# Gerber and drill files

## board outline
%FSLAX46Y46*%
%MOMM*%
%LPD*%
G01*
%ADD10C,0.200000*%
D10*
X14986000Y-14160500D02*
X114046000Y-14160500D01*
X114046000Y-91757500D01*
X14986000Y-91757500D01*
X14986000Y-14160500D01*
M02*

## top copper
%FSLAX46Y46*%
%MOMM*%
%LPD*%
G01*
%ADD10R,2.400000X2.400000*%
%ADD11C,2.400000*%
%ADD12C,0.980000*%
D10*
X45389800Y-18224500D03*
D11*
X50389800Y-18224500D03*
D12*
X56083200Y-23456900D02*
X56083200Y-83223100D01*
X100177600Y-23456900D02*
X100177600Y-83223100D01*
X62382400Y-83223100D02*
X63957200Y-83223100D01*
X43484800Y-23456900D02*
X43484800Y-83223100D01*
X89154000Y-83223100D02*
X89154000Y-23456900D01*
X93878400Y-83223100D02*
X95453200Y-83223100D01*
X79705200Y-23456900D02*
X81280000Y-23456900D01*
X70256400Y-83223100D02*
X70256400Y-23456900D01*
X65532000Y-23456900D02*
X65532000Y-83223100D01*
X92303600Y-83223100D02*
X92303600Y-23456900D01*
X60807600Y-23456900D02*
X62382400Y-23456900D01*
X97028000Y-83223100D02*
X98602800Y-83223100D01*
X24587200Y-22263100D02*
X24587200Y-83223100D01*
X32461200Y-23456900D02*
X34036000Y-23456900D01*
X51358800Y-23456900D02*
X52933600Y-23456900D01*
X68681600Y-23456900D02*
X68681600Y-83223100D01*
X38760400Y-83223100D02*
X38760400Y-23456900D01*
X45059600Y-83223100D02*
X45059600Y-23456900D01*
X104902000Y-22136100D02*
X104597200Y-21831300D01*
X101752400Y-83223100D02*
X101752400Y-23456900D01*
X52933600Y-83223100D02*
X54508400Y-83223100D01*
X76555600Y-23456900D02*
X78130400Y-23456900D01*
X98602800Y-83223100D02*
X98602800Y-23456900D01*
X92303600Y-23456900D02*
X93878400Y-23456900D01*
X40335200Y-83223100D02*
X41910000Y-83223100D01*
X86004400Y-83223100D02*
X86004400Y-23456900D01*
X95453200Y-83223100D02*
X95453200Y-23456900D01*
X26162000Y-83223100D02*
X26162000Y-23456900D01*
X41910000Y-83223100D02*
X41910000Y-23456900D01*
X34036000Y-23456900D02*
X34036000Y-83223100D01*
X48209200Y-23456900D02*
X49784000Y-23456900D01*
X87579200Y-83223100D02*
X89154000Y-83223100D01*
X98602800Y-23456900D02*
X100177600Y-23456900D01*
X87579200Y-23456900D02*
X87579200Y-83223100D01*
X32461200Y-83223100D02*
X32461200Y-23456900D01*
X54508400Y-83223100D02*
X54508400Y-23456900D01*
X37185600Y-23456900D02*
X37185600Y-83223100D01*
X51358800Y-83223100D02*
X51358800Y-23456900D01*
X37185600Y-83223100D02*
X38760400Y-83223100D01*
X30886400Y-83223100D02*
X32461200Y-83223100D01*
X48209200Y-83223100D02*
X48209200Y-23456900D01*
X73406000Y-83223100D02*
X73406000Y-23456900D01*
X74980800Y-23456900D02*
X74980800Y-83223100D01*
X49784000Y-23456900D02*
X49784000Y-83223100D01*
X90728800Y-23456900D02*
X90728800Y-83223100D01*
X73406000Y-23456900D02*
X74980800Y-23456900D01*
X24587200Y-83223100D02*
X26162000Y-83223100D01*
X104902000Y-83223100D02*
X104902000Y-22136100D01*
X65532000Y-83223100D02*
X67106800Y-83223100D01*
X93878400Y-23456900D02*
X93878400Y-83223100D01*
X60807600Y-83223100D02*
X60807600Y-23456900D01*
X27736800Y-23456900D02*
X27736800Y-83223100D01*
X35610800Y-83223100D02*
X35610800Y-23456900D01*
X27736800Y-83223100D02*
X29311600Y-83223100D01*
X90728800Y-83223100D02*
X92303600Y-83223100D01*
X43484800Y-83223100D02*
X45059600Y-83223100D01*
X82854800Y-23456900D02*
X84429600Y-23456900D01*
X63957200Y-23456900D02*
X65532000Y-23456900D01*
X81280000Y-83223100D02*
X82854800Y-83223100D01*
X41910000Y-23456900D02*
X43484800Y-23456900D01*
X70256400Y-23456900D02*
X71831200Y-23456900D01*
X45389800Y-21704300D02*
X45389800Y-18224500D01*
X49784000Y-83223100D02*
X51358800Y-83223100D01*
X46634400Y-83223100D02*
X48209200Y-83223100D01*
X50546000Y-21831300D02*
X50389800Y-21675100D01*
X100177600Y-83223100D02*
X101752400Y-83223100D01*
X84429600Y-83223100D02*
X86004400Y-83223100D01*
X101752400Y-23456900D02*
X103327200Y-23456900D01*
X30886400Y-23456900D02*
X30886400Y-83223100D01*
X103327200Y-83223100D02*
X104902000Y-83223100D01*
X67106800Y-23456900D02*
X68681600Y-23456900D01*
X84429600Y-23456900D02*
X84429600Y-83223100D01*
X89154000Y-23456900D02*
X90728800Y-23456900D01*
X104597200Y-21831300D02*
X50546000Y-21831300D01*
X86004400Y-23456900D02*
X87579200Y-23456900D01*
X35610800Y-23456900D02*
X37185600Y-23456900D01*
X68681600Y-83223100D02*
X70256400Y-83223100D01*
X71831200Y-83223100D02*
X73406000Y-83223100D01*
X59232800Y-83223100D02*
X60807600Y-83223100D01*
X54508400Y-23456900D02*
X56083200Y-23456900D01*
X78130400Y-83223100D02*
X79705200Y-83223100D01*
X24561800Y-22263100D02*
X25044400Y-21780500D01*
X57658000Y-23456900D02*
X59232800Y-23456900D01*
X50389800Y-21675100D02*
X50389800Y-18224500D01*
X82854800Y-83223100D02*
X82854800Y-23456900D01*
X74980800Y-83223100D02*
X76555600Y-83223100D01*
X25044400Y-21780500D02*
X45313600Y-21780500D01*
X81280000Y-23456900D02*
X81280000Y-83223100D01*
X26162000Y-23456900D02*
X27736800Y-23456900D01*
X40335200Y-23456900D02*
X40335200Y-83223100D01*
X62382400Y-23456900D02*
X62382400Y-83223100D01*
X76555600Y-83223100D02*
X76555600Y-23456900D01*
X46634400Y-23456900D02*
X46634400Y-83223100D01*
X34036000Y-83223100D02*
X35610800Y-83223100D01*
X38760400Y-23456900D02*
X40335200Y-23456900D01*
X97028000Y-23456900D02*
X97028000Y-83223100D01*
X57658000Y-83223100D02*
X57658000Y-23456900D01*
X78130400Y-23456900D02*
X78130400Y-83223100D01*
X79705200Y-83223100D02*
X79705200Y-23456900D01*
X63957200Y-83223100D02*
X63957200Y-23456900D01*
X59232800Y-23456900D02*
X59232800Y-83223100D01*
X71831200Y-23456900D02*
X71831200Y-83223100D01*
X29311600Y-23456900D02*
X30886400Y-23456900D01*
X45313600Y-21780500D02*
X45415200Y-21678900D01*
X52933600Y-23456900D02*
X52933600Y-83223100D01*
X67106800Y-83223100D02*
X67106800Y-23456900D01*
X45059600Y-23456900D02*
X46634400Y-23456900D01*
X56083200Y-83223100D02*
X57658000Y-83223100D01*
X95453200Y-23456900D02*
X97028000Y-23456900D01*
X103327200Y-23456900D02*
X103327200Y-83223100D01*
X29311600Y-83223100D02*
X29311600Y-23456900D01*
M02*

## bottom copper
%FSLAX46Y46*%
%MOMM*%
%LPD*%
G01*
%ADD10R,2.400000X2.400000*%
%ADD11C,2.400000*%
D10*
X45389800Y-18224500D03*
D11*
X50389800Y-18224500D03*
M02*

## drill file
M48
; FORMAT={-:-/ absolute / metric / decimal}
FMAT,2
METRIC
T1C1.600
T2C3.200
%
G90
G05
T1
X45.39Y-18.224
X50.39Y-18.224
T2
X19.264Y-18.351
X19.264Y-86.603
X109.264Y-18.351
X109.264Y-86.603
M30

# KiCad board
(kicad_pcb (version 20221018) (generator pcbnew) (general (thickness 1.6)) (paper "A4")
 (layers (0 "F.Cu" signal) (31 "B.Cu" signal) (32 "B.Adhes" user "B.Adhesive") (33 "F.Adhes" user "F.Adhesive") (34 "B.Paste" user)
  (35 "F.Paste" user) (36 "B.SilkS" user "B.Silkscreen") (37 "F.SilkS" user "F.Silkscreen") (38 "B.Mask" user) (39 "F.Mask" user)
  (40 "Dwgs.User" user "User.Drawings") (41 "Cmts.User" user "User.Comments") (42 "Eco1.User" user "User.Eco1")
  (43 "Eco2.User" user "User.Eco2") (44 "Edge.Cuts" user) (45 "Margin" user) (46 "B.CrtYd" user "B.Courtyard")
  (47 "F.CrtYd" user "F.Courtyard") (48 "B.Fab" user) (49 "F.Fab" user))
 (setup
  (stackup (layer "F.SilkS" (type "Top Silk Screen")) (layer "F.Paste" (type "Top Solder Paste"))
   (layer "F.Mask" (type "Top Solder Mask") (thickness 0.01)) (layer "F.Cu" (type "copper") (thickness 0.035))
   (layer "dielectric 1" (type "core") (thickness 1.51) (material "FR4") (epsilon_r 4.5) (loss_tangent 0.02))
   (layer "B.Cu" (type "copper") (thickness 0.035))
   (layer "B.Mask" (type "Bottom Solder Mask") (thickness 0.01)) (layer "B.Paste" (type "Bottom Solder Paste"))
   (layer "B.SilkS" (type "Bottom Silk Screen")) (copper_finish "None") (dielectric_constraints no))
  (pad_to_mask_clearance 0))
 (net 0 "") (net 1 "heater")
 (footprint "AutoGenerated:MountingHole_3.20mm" (layer "F.Cu") (at 99.264 70.6035)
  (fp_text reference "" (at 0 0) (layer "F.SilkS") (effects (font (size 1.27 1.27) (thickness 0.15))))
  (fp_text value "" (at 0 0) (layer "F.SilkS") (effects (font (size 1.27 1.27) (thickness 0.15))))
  (pad "" np_thru_hole circle (at 10 16) (size 3.2 3.2) (drill 3.2) (layers "F&B.Cu" "*.Mask")))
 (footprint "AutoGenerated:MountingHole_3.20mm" (layer "F.Cu") (at 19.264 18.3515)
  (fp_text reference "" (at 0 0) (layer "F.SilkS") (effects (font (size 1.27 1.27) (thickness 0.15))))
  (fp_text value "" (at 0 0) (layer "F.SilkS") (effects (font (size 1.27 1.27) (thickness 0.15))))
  (pad "" np_thru_hole circle (at 0 0) (size 3.2 3.2) (drill 3.2) (layers "*.Cu" "*.Mask")))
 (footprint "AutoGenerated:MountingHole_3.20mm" (layer "F.Cu") (at 99.264 18.3515)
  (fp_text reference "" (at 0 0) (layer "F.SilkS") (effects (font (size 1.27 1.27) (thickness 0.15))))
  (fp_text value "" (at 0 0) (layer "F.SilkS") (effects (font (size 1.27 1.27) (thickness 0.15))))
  (pad "" np_thru_hole circle (at 10 0) (size 3.2 3.2) (drill 3.2) (layers "F&B.Cu" "*.Mask")))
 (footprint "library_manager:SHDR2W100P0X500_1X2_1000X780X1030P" (layer "F.Cu") (at 45.3898 18.2245)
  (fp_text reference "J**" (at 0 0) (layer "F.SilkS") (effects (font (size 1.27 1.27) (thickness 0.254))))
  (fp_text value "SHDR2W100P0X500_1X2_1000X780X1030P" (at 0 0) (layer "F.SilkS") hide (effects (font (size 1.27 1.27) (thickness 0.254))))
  (pad "1" thru_hole rect (at 0 0) (size 2.4 2.4) (drill 1.6) (layers "*.Cu" "*.Mask") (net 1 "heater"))
  (pad "2" thru_hole circle (at 5 0) (size 2.4 2.4) (drill 1.6) (layers "*.Cu" "*.Mask") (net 1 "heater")))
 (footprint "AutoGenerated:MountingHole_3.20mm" (layer "F.Cu") (at 19.264 70.6035)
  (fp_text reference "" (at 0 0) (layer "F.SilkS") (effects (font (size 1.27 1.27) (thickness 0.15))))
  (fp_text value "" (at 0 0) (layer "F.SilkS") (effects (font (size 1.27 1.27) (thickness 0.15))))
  (pad "" np_thru_hole circle (at 0 16) (size 3.2 3.2) (drill 3.2) (layers "F&B.Cu" "*.Mask")))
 (gr_rect (start 14.986 14.1605) (end 114.046 91.7575) (stroke (width 0.2) (type solid)) (fill none) (layer "Edge.Cuts"))
 (segment (start 56.0832 23.4569) (end 56.0832 83.2231) (width 0.98) (layer "F.Cu") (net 1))
 (segment (start 100.1776 23.4569) (end 100.1776 83.2231) (width 0.98) (layer "F.Cu") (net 1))
 (segment (start 62.3824 83.2231) (end 63.9572 83.2231) (width 0.98) (layer "F.Cu") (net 1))
 (segment (start 43.4848 23.4569) (end 43.4848 83.2231) (width 0.98) (layer "F.Cu") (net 1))
 (segment (start 89.154 83.2231) (end 89.154 23.4569) (width 0.98) (layer "F.Cu") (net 1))
 (segment (start 93.8784 83.2231) (end 95.4532 83.2231) (width 0.98) (layer "F.Cu") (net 1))
 (segment (start 79.7052 23.4569) (end 81.28 23.4569) (width 0.98) (layer "F.Cu") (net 1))
 (segment (start 70.2564 83.2231) (end 70.2564 23.4569) (width 0.98) (layer "F.Cu") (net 1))
 (segment (start 65.532 23.4569) (end 65.532 83.2231) (width 0.98) (layer "F.Cu") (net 1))
 (segment (start 92.3036 83.2231) (end 92.3036 23.4569) (width 0.98) (layer "F.Cu") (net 1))
 (segment (start 60.8076 23.4569) (end 62.3824 23.4569) (width 0.98) (layer "F.Cu") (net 1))
 (segment (start 97.028 83.2231) (end 98.6028 83.2231) (width 0.98) (layer "F.Cu") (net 1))
 (segment (start 24.5872 22.2631) (end 24.5872 83.2231) (width 0.98) (layer "F.Cu") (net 1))
 (segment (start 32.4612 23.4569) (end 34.036 23.4569) (width 0.98) (layer "F.Cu") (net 1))
 (segment (start 51.3588 23.4569) (end 52.9336 23.4569) (width 0.98) (layer "F.Cu") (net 1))
 (segment (start 68.6816 23.4569) (end 68.6816 83.2231) (width 0.98) (layer "F.Cu") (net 1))
 (segment (start 38.7604 83.2231) (end 38.7604 23.4569) (width 0.98) (layer "F.Cu") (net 1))
 (segment (start 45.0596 83.2231) (end 45.0596 23.4569) (width 0.98) (layer "F.Cu") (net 1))
 (segment (start 104.902 22.1361) (end 104.5972 21.8313) (width 0.98) (layer "F.Cu") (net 1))
 (segment (start 101.7524 83.2231) (end 101.7524 23.4569) (width 0.98) (layer "F.Cu") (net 1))
 (segment (start 52.9336 83.2231) (end 54.5084 83.2231) (width 0.98) (layer "F.Cu") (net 1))
 (segment (start 76.5556 23.4569) (end 78.1304 23.4569) (width 0.98) (layer "F.Cu") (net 1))
 (segment (start 98.6028 83.2231) (end 98.6028 23.4569) (width 0.98) (layer "F.Cu") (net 1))
 (segment (start 92.3036 23.4569) (end 93.8784 23.4569) (width 0.98) (layer "F.Cu") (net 1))
 (segment (start 40.3352 83.2231) (end 41.91 83.2231) (width 0.98) (layer "F.Cu") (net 1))
 (segment (start 86.0044 83.2231) (end 86.0044 23.4569) (width 0.98) (layer "F.Cu") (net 1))
 (segment (start 95.4532 83.2231) (end 95.4532 23.4569) (width 0.98) (layer "F.Cu") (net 1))
 (segment (start 26.162 83.2231) (end 26.162 23.4569) (width 0.98) (layer "F.Cu") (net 1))
 (segment (start 41.91 83.2231) (end 41.91 23.4569) (width 0.98) (layer "F.Cu") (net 1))
 (segment (start 34.036 23.4569) (end 34.036 83.2231) (width 0.98) (layer "F.Cu") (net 1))
 (segment (start 48.2092 23.4569) (end 49.784 23.4569) (width 0.98) (layer "F.Cu") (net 1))
 (segment (start 87.5792 83.2231) (end 89.154 83.2231) (width 0.98) (layer "F.Cu") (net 1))
 (segment (start 98.6028 23.4569) (end 100.1776 23.4569) (width 0.98) (layer "F.Cu") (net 1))
 (segment (start 87.5792 23.4569) (end 87.5792 83.2231) (width 0.98) (layer "F.Cu") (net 1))
 (segment (start 32.4612 83.2231) (end 32.4612 23.4569) (width 0.98) (layer "F.Cu") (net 1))
 (segment (start 54.5084 83.2231) (end 54.5084 23.4569) (width 0.98) (layer "F.Cu") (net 1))
 (segment (start 37.1856 23.4569) (end 37.1856 83.2231) (width 0.98) (layer "F.Cu") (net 1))
 (segment (start 51.3588 83.2231) (end 51.3588 23.4569) (width 0.98) (layer "F.Cu") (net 1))
 (segment (start 37.1856 83.2231) (end 38.7604 83.2231) (width 0.98) (layer "F.Cu") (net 1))
 (segment (start 30.8864 83.2231) (end 32.4612 83.2231) (width 0.98) (layer "F.Cu") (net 1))
 (segment (start 48.2092 83.2231) (end 48.2092 23.4569) (width 0.98) (layer "F.Cu") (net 1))
 (segment (start 73.406 83.2231) (end 73.406 23.4569) (width 0.98) (layer "F.Cu") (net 1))
 (segment (start 74.9808 23.4569) (end 74.9808 83.2231) (width 0.98) (layer "F.Cu") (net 1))
 (segment (start 49.784 23.4569) (end 49.784 83.2231) (width 0.98) (layer "F.Cu") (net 1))
 (segment (start 90.7288 23.4569) (end 90.7288 83.2231) (width 0.98) (layer "F.Cu") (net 1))
 (segment (start 73.406 23.4569) (end 74.9808 23.4569) (width 0.98) (layer "F.Cu") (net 1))
 (segment (start 24.5872 83.2231) (end 26.162 83.2231) (width 0.98) (layer "F.Cu") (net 1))
 (segment (start 104.902 83.2231) (end 104.902 22.1361) (width 0.98) (layer "F.Cu") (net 1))
 (segment (start 65.532 83.2231) (end 67.1068 83.2231) (width 0.98) (layer "F.Cu") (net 1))
 (segment (start 93.8784 23.4569) (end 93.8784 83.2231) (width 0.98) (layer "F.Cu") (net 1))
 (segment (start 60.8076 83.2231) (end 60.8076 23.4569) (width 0.98) (layer "F.Cu") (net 1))
 (segment (start 27.7368 23.4569) (end 27.7368 83.2231) (width 0.98) (layer "F.Cu") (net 1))
 (segment (start 35.6108 83.2231) (end 35.6108 23.4569) (width 0.98) (layer "F.Cu") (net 1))
 (segment (start 27.7368 83.2231) (end 29.3116 83.2231) (width 0.98) (layer "F.Cu") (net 1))
 (segment (start 90.7288 83.2231) (end 92.3036 83.2231) (width 0.98) (layer "F.Cu") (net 1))
 (segment (start 43.4848 83.2231) (end 45.0596 83.2231) (width 0.98) (layer "F.Cu") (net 1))
 (segment (start 82.8548 23.4569) (end 84.4296 23.4569) (width 0.98) (layer "F.Cu") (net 1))
 (segment (start 63.9572 23.4569) (end 65.532 23.4569) (width 0.98) (layer "F.Cu") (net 1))
 (segment (start 81.28 83.2231) (end 82.8548 83.2231) (width 0.98) (layer "F.Cu") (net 1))
 (segment (start 41.91 23.4569) (end 43.4848 23.4569) (width 0.98) (layer "F.Cu") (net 1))
 (segment (start 70.2564 23.4569) (end 71.8312 23.4569) (width 0.98) (layer "F.Cu") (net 1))
 (segment (start 45.3898 21.7043) (end 45.3898 18.2245) (width 0.98) (layer "F.Cu") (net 1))
 (segment (start 49.784 83.2231) (end 51.3588 83.2231) (width 0.98) (layer "F.Cu") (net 1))
 (segment (start 46.6344 83.2231) (end 48.2092 83.2231) (width 0.98) (layer "F.Cu") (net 1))
 (segment (start 50.546 21.8313) (end 50.3898 21.6751) (width 0.98) (layer "F.Cu") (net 1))
 (segment (start 100.1776 83.2231) (end 101.7524 83.2231) (width 0.98) (layer "F.Cu") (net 1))
 (segment (start 84.4296 83.2231) (end 86.0044 83.2231) (width 0.98) (layer "F.Cu") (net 1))
 (segment (start 101.7524 23.4569) (end 103.3272 23.4569) (width 0.98) (layer "F.Cu") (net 1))
 (segment (start 30.8864 23.4569) (end 30.8864 83.2231) (width 0.98) (layer "F.Cu") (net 1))
 (segment (start 103.3272 83.2231) (end 104.902 83.2231) (width 0.98) (layer "F.Cu") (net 1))
 (segment (start 67.1068 23.4569) (end 68.6816 23.4569) (width 0.98) (layer "F.Cu") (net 1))
 (segment (start 84.4296 23.4569) (end 84.4296 83.2231) (width 0.98) (layer "F.Cu") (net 1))
 (segment (start 89.154 23.4569) (end 90.7288 23.4569) (width 0.98) (layer "F.Cu") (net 1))
 (segment (start 104.5972 21.8313) (end 50.546 21.8313) (width 0.98) (layer "F.Cu") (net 1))
 (segment (start 86.0044 23.4569) (end 87.5792 23.4569) (width 0.98) (layer "F.Cu") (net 1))
 (segment (start 35.6108 23.4569) (end 37.1856 23.4569) (width 0.98) (layer "F.Cu") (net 1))
 (segment (start 68.6816 83.2231) (end 70.2564 83.2231) (width 0.98) (layer "F.Cu") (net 1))
 (segment (start 71.8312 83.2231) (end 73.406 83.2231) (width 0.98) (layer "F.Cu") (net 1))
 (segment (start 59.2328 83.2231) (end 60.8076 83.2231) (width 0.98) (layer "F.Cu") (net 1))
 (segment (start 54.5084 23.4569) (end 56.0832 23.4569) (width 0.98) (layer "F.Cu") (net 1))
 (segment (start 78.1304 83.2231) (end 79.7052 83.2231) (width 0.98) (layer "F.Cu") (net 1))
 (segment (start 24.5618 22.2631) (end 25.0444 21.7805) (width 0.98) (layer "F.Cu") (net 1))
 (segment (start 57.658 23.4569) (end 59.2328 23.4569) (width 0.98) (layer "F.Cu") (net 1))
 (segment (start 50.3898 21.6751) (end 50.3898 18.2245) (width 0.98) (layer "F.Cu") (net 1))
 (segment (start 82.8548 83.2231) (end 82.8548 23.4569) (width 0.98) (layer "F.Cu") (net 1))
 (segment (start 74.9808 83.2231) (end 76.5556 83.2231) (width 0.98) (layer "F.Cu") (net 1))
 (segment (start 25.0444 21.7805) (end 45.3136 21.7805) (width 0.98) (layer "F.Cu") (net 1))
 (segment (start 81.28 23.4569) (end 81.28 83.2231) (width 0.98) (layer "F.Cu") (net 1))
 (segment (start 26.162 23.4569) (end 27.7368 23.4569) (width 0.98) (layer "F.Cu") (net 1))
 (segment (start 40.3352 23.4569) (end 40.3352 83.2231) (width 0.98) (layer "F.Cu") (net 1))
 (segment (start 62.3824 23.4569) (end 62.3824 83.2231) (width 0.98) (layer "F.Cu") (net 1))
 (segment (start 76.5556 83.2231) (end 76.5556 23.4569) (width 0.98) (layer "F.Cu") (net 1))
 (segment (start 46.6344 23.4569) (end 46.6344 83.2231) (width 0.98) (layer "F.Cu") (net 1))
 (segment (start 34.036 83.2231) (end 35.6108 83.2231) (width 0.98) (layer "F.Cu") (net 1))
 (segment (start 38.7604 23.4569) (end 40.3352 23.4569) (width 0.98) (layer "F.Cu") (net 1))
 (segment (start 97.028 23.4569) (end 97.028 83.2231) (width 0.98) (layer "F.Cu") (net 1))
 (segment (start 57.658 83.2231) (end 57.658 23.4569) (width 0.98) (layer "F.Cu") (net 1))
 (segment (start 78.1304 23.4569) (end 78.1304 83.2231) (width 0.98) (layer "F.Cu") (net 1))
 (segment (start 79.7052 83.2231) (end 79.7052 23.4569) (width 0.98) (layer "F.Cu") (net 1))
 (segment (start 63.9572 83.2231) (end 63.9572 23.4569) (width 0.98) (layer "F.Cu") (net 1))
 (segment (start 59.2328 23.4569) (end 59.2328 83.2231) (width 0.98) (layer "F.Cu") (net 1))
 (segment (start 71.8312 23.4569) (end 71.8312 83.2231) (width 0.98) (layer "F.Cu") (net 1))
 (segment (start 29.3116 23.4569) (end 30.8864 23.4569) (width 0.98) (layer "F.Cu") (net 1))
 (segment (start 45.3136 21.7805) (end 45.4152 21.6789) (width 0.98) (layer "F.Cu") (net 1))
 (segment (start 52.9336 23.4569) (end 52.9336 83.2231) (width 0.98) (layer "F.Cu") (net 1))
 (segment (start 67.1068 83.2231) (end 67.1068 23.4569) (width 0.98) (layer "F.Cu") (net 1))
 (segment (start 45.0596 23.4569) (end 46.6344 23.4569) (width 0.98) (layer "F.Cu") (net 1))
 (segment (start 56.0832 83.2231) (end 57.658 83.2231) (width 0.98) (layer "F.Cu") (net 1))
 (segment (start 95.4532 23.4569) (end 97.028 23.4569) (width 0.98) (layer "F.Cu") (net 1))
 (segment (start 103.3272 23.4569) (end 103.3272 83.2231) (width 0.98) (layer "F.Cu") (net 1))
 (segment (start 29.3116 83.2231) (end 29.3116 23.4569) (width 0.98) (layer "F.Cu") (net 1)))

